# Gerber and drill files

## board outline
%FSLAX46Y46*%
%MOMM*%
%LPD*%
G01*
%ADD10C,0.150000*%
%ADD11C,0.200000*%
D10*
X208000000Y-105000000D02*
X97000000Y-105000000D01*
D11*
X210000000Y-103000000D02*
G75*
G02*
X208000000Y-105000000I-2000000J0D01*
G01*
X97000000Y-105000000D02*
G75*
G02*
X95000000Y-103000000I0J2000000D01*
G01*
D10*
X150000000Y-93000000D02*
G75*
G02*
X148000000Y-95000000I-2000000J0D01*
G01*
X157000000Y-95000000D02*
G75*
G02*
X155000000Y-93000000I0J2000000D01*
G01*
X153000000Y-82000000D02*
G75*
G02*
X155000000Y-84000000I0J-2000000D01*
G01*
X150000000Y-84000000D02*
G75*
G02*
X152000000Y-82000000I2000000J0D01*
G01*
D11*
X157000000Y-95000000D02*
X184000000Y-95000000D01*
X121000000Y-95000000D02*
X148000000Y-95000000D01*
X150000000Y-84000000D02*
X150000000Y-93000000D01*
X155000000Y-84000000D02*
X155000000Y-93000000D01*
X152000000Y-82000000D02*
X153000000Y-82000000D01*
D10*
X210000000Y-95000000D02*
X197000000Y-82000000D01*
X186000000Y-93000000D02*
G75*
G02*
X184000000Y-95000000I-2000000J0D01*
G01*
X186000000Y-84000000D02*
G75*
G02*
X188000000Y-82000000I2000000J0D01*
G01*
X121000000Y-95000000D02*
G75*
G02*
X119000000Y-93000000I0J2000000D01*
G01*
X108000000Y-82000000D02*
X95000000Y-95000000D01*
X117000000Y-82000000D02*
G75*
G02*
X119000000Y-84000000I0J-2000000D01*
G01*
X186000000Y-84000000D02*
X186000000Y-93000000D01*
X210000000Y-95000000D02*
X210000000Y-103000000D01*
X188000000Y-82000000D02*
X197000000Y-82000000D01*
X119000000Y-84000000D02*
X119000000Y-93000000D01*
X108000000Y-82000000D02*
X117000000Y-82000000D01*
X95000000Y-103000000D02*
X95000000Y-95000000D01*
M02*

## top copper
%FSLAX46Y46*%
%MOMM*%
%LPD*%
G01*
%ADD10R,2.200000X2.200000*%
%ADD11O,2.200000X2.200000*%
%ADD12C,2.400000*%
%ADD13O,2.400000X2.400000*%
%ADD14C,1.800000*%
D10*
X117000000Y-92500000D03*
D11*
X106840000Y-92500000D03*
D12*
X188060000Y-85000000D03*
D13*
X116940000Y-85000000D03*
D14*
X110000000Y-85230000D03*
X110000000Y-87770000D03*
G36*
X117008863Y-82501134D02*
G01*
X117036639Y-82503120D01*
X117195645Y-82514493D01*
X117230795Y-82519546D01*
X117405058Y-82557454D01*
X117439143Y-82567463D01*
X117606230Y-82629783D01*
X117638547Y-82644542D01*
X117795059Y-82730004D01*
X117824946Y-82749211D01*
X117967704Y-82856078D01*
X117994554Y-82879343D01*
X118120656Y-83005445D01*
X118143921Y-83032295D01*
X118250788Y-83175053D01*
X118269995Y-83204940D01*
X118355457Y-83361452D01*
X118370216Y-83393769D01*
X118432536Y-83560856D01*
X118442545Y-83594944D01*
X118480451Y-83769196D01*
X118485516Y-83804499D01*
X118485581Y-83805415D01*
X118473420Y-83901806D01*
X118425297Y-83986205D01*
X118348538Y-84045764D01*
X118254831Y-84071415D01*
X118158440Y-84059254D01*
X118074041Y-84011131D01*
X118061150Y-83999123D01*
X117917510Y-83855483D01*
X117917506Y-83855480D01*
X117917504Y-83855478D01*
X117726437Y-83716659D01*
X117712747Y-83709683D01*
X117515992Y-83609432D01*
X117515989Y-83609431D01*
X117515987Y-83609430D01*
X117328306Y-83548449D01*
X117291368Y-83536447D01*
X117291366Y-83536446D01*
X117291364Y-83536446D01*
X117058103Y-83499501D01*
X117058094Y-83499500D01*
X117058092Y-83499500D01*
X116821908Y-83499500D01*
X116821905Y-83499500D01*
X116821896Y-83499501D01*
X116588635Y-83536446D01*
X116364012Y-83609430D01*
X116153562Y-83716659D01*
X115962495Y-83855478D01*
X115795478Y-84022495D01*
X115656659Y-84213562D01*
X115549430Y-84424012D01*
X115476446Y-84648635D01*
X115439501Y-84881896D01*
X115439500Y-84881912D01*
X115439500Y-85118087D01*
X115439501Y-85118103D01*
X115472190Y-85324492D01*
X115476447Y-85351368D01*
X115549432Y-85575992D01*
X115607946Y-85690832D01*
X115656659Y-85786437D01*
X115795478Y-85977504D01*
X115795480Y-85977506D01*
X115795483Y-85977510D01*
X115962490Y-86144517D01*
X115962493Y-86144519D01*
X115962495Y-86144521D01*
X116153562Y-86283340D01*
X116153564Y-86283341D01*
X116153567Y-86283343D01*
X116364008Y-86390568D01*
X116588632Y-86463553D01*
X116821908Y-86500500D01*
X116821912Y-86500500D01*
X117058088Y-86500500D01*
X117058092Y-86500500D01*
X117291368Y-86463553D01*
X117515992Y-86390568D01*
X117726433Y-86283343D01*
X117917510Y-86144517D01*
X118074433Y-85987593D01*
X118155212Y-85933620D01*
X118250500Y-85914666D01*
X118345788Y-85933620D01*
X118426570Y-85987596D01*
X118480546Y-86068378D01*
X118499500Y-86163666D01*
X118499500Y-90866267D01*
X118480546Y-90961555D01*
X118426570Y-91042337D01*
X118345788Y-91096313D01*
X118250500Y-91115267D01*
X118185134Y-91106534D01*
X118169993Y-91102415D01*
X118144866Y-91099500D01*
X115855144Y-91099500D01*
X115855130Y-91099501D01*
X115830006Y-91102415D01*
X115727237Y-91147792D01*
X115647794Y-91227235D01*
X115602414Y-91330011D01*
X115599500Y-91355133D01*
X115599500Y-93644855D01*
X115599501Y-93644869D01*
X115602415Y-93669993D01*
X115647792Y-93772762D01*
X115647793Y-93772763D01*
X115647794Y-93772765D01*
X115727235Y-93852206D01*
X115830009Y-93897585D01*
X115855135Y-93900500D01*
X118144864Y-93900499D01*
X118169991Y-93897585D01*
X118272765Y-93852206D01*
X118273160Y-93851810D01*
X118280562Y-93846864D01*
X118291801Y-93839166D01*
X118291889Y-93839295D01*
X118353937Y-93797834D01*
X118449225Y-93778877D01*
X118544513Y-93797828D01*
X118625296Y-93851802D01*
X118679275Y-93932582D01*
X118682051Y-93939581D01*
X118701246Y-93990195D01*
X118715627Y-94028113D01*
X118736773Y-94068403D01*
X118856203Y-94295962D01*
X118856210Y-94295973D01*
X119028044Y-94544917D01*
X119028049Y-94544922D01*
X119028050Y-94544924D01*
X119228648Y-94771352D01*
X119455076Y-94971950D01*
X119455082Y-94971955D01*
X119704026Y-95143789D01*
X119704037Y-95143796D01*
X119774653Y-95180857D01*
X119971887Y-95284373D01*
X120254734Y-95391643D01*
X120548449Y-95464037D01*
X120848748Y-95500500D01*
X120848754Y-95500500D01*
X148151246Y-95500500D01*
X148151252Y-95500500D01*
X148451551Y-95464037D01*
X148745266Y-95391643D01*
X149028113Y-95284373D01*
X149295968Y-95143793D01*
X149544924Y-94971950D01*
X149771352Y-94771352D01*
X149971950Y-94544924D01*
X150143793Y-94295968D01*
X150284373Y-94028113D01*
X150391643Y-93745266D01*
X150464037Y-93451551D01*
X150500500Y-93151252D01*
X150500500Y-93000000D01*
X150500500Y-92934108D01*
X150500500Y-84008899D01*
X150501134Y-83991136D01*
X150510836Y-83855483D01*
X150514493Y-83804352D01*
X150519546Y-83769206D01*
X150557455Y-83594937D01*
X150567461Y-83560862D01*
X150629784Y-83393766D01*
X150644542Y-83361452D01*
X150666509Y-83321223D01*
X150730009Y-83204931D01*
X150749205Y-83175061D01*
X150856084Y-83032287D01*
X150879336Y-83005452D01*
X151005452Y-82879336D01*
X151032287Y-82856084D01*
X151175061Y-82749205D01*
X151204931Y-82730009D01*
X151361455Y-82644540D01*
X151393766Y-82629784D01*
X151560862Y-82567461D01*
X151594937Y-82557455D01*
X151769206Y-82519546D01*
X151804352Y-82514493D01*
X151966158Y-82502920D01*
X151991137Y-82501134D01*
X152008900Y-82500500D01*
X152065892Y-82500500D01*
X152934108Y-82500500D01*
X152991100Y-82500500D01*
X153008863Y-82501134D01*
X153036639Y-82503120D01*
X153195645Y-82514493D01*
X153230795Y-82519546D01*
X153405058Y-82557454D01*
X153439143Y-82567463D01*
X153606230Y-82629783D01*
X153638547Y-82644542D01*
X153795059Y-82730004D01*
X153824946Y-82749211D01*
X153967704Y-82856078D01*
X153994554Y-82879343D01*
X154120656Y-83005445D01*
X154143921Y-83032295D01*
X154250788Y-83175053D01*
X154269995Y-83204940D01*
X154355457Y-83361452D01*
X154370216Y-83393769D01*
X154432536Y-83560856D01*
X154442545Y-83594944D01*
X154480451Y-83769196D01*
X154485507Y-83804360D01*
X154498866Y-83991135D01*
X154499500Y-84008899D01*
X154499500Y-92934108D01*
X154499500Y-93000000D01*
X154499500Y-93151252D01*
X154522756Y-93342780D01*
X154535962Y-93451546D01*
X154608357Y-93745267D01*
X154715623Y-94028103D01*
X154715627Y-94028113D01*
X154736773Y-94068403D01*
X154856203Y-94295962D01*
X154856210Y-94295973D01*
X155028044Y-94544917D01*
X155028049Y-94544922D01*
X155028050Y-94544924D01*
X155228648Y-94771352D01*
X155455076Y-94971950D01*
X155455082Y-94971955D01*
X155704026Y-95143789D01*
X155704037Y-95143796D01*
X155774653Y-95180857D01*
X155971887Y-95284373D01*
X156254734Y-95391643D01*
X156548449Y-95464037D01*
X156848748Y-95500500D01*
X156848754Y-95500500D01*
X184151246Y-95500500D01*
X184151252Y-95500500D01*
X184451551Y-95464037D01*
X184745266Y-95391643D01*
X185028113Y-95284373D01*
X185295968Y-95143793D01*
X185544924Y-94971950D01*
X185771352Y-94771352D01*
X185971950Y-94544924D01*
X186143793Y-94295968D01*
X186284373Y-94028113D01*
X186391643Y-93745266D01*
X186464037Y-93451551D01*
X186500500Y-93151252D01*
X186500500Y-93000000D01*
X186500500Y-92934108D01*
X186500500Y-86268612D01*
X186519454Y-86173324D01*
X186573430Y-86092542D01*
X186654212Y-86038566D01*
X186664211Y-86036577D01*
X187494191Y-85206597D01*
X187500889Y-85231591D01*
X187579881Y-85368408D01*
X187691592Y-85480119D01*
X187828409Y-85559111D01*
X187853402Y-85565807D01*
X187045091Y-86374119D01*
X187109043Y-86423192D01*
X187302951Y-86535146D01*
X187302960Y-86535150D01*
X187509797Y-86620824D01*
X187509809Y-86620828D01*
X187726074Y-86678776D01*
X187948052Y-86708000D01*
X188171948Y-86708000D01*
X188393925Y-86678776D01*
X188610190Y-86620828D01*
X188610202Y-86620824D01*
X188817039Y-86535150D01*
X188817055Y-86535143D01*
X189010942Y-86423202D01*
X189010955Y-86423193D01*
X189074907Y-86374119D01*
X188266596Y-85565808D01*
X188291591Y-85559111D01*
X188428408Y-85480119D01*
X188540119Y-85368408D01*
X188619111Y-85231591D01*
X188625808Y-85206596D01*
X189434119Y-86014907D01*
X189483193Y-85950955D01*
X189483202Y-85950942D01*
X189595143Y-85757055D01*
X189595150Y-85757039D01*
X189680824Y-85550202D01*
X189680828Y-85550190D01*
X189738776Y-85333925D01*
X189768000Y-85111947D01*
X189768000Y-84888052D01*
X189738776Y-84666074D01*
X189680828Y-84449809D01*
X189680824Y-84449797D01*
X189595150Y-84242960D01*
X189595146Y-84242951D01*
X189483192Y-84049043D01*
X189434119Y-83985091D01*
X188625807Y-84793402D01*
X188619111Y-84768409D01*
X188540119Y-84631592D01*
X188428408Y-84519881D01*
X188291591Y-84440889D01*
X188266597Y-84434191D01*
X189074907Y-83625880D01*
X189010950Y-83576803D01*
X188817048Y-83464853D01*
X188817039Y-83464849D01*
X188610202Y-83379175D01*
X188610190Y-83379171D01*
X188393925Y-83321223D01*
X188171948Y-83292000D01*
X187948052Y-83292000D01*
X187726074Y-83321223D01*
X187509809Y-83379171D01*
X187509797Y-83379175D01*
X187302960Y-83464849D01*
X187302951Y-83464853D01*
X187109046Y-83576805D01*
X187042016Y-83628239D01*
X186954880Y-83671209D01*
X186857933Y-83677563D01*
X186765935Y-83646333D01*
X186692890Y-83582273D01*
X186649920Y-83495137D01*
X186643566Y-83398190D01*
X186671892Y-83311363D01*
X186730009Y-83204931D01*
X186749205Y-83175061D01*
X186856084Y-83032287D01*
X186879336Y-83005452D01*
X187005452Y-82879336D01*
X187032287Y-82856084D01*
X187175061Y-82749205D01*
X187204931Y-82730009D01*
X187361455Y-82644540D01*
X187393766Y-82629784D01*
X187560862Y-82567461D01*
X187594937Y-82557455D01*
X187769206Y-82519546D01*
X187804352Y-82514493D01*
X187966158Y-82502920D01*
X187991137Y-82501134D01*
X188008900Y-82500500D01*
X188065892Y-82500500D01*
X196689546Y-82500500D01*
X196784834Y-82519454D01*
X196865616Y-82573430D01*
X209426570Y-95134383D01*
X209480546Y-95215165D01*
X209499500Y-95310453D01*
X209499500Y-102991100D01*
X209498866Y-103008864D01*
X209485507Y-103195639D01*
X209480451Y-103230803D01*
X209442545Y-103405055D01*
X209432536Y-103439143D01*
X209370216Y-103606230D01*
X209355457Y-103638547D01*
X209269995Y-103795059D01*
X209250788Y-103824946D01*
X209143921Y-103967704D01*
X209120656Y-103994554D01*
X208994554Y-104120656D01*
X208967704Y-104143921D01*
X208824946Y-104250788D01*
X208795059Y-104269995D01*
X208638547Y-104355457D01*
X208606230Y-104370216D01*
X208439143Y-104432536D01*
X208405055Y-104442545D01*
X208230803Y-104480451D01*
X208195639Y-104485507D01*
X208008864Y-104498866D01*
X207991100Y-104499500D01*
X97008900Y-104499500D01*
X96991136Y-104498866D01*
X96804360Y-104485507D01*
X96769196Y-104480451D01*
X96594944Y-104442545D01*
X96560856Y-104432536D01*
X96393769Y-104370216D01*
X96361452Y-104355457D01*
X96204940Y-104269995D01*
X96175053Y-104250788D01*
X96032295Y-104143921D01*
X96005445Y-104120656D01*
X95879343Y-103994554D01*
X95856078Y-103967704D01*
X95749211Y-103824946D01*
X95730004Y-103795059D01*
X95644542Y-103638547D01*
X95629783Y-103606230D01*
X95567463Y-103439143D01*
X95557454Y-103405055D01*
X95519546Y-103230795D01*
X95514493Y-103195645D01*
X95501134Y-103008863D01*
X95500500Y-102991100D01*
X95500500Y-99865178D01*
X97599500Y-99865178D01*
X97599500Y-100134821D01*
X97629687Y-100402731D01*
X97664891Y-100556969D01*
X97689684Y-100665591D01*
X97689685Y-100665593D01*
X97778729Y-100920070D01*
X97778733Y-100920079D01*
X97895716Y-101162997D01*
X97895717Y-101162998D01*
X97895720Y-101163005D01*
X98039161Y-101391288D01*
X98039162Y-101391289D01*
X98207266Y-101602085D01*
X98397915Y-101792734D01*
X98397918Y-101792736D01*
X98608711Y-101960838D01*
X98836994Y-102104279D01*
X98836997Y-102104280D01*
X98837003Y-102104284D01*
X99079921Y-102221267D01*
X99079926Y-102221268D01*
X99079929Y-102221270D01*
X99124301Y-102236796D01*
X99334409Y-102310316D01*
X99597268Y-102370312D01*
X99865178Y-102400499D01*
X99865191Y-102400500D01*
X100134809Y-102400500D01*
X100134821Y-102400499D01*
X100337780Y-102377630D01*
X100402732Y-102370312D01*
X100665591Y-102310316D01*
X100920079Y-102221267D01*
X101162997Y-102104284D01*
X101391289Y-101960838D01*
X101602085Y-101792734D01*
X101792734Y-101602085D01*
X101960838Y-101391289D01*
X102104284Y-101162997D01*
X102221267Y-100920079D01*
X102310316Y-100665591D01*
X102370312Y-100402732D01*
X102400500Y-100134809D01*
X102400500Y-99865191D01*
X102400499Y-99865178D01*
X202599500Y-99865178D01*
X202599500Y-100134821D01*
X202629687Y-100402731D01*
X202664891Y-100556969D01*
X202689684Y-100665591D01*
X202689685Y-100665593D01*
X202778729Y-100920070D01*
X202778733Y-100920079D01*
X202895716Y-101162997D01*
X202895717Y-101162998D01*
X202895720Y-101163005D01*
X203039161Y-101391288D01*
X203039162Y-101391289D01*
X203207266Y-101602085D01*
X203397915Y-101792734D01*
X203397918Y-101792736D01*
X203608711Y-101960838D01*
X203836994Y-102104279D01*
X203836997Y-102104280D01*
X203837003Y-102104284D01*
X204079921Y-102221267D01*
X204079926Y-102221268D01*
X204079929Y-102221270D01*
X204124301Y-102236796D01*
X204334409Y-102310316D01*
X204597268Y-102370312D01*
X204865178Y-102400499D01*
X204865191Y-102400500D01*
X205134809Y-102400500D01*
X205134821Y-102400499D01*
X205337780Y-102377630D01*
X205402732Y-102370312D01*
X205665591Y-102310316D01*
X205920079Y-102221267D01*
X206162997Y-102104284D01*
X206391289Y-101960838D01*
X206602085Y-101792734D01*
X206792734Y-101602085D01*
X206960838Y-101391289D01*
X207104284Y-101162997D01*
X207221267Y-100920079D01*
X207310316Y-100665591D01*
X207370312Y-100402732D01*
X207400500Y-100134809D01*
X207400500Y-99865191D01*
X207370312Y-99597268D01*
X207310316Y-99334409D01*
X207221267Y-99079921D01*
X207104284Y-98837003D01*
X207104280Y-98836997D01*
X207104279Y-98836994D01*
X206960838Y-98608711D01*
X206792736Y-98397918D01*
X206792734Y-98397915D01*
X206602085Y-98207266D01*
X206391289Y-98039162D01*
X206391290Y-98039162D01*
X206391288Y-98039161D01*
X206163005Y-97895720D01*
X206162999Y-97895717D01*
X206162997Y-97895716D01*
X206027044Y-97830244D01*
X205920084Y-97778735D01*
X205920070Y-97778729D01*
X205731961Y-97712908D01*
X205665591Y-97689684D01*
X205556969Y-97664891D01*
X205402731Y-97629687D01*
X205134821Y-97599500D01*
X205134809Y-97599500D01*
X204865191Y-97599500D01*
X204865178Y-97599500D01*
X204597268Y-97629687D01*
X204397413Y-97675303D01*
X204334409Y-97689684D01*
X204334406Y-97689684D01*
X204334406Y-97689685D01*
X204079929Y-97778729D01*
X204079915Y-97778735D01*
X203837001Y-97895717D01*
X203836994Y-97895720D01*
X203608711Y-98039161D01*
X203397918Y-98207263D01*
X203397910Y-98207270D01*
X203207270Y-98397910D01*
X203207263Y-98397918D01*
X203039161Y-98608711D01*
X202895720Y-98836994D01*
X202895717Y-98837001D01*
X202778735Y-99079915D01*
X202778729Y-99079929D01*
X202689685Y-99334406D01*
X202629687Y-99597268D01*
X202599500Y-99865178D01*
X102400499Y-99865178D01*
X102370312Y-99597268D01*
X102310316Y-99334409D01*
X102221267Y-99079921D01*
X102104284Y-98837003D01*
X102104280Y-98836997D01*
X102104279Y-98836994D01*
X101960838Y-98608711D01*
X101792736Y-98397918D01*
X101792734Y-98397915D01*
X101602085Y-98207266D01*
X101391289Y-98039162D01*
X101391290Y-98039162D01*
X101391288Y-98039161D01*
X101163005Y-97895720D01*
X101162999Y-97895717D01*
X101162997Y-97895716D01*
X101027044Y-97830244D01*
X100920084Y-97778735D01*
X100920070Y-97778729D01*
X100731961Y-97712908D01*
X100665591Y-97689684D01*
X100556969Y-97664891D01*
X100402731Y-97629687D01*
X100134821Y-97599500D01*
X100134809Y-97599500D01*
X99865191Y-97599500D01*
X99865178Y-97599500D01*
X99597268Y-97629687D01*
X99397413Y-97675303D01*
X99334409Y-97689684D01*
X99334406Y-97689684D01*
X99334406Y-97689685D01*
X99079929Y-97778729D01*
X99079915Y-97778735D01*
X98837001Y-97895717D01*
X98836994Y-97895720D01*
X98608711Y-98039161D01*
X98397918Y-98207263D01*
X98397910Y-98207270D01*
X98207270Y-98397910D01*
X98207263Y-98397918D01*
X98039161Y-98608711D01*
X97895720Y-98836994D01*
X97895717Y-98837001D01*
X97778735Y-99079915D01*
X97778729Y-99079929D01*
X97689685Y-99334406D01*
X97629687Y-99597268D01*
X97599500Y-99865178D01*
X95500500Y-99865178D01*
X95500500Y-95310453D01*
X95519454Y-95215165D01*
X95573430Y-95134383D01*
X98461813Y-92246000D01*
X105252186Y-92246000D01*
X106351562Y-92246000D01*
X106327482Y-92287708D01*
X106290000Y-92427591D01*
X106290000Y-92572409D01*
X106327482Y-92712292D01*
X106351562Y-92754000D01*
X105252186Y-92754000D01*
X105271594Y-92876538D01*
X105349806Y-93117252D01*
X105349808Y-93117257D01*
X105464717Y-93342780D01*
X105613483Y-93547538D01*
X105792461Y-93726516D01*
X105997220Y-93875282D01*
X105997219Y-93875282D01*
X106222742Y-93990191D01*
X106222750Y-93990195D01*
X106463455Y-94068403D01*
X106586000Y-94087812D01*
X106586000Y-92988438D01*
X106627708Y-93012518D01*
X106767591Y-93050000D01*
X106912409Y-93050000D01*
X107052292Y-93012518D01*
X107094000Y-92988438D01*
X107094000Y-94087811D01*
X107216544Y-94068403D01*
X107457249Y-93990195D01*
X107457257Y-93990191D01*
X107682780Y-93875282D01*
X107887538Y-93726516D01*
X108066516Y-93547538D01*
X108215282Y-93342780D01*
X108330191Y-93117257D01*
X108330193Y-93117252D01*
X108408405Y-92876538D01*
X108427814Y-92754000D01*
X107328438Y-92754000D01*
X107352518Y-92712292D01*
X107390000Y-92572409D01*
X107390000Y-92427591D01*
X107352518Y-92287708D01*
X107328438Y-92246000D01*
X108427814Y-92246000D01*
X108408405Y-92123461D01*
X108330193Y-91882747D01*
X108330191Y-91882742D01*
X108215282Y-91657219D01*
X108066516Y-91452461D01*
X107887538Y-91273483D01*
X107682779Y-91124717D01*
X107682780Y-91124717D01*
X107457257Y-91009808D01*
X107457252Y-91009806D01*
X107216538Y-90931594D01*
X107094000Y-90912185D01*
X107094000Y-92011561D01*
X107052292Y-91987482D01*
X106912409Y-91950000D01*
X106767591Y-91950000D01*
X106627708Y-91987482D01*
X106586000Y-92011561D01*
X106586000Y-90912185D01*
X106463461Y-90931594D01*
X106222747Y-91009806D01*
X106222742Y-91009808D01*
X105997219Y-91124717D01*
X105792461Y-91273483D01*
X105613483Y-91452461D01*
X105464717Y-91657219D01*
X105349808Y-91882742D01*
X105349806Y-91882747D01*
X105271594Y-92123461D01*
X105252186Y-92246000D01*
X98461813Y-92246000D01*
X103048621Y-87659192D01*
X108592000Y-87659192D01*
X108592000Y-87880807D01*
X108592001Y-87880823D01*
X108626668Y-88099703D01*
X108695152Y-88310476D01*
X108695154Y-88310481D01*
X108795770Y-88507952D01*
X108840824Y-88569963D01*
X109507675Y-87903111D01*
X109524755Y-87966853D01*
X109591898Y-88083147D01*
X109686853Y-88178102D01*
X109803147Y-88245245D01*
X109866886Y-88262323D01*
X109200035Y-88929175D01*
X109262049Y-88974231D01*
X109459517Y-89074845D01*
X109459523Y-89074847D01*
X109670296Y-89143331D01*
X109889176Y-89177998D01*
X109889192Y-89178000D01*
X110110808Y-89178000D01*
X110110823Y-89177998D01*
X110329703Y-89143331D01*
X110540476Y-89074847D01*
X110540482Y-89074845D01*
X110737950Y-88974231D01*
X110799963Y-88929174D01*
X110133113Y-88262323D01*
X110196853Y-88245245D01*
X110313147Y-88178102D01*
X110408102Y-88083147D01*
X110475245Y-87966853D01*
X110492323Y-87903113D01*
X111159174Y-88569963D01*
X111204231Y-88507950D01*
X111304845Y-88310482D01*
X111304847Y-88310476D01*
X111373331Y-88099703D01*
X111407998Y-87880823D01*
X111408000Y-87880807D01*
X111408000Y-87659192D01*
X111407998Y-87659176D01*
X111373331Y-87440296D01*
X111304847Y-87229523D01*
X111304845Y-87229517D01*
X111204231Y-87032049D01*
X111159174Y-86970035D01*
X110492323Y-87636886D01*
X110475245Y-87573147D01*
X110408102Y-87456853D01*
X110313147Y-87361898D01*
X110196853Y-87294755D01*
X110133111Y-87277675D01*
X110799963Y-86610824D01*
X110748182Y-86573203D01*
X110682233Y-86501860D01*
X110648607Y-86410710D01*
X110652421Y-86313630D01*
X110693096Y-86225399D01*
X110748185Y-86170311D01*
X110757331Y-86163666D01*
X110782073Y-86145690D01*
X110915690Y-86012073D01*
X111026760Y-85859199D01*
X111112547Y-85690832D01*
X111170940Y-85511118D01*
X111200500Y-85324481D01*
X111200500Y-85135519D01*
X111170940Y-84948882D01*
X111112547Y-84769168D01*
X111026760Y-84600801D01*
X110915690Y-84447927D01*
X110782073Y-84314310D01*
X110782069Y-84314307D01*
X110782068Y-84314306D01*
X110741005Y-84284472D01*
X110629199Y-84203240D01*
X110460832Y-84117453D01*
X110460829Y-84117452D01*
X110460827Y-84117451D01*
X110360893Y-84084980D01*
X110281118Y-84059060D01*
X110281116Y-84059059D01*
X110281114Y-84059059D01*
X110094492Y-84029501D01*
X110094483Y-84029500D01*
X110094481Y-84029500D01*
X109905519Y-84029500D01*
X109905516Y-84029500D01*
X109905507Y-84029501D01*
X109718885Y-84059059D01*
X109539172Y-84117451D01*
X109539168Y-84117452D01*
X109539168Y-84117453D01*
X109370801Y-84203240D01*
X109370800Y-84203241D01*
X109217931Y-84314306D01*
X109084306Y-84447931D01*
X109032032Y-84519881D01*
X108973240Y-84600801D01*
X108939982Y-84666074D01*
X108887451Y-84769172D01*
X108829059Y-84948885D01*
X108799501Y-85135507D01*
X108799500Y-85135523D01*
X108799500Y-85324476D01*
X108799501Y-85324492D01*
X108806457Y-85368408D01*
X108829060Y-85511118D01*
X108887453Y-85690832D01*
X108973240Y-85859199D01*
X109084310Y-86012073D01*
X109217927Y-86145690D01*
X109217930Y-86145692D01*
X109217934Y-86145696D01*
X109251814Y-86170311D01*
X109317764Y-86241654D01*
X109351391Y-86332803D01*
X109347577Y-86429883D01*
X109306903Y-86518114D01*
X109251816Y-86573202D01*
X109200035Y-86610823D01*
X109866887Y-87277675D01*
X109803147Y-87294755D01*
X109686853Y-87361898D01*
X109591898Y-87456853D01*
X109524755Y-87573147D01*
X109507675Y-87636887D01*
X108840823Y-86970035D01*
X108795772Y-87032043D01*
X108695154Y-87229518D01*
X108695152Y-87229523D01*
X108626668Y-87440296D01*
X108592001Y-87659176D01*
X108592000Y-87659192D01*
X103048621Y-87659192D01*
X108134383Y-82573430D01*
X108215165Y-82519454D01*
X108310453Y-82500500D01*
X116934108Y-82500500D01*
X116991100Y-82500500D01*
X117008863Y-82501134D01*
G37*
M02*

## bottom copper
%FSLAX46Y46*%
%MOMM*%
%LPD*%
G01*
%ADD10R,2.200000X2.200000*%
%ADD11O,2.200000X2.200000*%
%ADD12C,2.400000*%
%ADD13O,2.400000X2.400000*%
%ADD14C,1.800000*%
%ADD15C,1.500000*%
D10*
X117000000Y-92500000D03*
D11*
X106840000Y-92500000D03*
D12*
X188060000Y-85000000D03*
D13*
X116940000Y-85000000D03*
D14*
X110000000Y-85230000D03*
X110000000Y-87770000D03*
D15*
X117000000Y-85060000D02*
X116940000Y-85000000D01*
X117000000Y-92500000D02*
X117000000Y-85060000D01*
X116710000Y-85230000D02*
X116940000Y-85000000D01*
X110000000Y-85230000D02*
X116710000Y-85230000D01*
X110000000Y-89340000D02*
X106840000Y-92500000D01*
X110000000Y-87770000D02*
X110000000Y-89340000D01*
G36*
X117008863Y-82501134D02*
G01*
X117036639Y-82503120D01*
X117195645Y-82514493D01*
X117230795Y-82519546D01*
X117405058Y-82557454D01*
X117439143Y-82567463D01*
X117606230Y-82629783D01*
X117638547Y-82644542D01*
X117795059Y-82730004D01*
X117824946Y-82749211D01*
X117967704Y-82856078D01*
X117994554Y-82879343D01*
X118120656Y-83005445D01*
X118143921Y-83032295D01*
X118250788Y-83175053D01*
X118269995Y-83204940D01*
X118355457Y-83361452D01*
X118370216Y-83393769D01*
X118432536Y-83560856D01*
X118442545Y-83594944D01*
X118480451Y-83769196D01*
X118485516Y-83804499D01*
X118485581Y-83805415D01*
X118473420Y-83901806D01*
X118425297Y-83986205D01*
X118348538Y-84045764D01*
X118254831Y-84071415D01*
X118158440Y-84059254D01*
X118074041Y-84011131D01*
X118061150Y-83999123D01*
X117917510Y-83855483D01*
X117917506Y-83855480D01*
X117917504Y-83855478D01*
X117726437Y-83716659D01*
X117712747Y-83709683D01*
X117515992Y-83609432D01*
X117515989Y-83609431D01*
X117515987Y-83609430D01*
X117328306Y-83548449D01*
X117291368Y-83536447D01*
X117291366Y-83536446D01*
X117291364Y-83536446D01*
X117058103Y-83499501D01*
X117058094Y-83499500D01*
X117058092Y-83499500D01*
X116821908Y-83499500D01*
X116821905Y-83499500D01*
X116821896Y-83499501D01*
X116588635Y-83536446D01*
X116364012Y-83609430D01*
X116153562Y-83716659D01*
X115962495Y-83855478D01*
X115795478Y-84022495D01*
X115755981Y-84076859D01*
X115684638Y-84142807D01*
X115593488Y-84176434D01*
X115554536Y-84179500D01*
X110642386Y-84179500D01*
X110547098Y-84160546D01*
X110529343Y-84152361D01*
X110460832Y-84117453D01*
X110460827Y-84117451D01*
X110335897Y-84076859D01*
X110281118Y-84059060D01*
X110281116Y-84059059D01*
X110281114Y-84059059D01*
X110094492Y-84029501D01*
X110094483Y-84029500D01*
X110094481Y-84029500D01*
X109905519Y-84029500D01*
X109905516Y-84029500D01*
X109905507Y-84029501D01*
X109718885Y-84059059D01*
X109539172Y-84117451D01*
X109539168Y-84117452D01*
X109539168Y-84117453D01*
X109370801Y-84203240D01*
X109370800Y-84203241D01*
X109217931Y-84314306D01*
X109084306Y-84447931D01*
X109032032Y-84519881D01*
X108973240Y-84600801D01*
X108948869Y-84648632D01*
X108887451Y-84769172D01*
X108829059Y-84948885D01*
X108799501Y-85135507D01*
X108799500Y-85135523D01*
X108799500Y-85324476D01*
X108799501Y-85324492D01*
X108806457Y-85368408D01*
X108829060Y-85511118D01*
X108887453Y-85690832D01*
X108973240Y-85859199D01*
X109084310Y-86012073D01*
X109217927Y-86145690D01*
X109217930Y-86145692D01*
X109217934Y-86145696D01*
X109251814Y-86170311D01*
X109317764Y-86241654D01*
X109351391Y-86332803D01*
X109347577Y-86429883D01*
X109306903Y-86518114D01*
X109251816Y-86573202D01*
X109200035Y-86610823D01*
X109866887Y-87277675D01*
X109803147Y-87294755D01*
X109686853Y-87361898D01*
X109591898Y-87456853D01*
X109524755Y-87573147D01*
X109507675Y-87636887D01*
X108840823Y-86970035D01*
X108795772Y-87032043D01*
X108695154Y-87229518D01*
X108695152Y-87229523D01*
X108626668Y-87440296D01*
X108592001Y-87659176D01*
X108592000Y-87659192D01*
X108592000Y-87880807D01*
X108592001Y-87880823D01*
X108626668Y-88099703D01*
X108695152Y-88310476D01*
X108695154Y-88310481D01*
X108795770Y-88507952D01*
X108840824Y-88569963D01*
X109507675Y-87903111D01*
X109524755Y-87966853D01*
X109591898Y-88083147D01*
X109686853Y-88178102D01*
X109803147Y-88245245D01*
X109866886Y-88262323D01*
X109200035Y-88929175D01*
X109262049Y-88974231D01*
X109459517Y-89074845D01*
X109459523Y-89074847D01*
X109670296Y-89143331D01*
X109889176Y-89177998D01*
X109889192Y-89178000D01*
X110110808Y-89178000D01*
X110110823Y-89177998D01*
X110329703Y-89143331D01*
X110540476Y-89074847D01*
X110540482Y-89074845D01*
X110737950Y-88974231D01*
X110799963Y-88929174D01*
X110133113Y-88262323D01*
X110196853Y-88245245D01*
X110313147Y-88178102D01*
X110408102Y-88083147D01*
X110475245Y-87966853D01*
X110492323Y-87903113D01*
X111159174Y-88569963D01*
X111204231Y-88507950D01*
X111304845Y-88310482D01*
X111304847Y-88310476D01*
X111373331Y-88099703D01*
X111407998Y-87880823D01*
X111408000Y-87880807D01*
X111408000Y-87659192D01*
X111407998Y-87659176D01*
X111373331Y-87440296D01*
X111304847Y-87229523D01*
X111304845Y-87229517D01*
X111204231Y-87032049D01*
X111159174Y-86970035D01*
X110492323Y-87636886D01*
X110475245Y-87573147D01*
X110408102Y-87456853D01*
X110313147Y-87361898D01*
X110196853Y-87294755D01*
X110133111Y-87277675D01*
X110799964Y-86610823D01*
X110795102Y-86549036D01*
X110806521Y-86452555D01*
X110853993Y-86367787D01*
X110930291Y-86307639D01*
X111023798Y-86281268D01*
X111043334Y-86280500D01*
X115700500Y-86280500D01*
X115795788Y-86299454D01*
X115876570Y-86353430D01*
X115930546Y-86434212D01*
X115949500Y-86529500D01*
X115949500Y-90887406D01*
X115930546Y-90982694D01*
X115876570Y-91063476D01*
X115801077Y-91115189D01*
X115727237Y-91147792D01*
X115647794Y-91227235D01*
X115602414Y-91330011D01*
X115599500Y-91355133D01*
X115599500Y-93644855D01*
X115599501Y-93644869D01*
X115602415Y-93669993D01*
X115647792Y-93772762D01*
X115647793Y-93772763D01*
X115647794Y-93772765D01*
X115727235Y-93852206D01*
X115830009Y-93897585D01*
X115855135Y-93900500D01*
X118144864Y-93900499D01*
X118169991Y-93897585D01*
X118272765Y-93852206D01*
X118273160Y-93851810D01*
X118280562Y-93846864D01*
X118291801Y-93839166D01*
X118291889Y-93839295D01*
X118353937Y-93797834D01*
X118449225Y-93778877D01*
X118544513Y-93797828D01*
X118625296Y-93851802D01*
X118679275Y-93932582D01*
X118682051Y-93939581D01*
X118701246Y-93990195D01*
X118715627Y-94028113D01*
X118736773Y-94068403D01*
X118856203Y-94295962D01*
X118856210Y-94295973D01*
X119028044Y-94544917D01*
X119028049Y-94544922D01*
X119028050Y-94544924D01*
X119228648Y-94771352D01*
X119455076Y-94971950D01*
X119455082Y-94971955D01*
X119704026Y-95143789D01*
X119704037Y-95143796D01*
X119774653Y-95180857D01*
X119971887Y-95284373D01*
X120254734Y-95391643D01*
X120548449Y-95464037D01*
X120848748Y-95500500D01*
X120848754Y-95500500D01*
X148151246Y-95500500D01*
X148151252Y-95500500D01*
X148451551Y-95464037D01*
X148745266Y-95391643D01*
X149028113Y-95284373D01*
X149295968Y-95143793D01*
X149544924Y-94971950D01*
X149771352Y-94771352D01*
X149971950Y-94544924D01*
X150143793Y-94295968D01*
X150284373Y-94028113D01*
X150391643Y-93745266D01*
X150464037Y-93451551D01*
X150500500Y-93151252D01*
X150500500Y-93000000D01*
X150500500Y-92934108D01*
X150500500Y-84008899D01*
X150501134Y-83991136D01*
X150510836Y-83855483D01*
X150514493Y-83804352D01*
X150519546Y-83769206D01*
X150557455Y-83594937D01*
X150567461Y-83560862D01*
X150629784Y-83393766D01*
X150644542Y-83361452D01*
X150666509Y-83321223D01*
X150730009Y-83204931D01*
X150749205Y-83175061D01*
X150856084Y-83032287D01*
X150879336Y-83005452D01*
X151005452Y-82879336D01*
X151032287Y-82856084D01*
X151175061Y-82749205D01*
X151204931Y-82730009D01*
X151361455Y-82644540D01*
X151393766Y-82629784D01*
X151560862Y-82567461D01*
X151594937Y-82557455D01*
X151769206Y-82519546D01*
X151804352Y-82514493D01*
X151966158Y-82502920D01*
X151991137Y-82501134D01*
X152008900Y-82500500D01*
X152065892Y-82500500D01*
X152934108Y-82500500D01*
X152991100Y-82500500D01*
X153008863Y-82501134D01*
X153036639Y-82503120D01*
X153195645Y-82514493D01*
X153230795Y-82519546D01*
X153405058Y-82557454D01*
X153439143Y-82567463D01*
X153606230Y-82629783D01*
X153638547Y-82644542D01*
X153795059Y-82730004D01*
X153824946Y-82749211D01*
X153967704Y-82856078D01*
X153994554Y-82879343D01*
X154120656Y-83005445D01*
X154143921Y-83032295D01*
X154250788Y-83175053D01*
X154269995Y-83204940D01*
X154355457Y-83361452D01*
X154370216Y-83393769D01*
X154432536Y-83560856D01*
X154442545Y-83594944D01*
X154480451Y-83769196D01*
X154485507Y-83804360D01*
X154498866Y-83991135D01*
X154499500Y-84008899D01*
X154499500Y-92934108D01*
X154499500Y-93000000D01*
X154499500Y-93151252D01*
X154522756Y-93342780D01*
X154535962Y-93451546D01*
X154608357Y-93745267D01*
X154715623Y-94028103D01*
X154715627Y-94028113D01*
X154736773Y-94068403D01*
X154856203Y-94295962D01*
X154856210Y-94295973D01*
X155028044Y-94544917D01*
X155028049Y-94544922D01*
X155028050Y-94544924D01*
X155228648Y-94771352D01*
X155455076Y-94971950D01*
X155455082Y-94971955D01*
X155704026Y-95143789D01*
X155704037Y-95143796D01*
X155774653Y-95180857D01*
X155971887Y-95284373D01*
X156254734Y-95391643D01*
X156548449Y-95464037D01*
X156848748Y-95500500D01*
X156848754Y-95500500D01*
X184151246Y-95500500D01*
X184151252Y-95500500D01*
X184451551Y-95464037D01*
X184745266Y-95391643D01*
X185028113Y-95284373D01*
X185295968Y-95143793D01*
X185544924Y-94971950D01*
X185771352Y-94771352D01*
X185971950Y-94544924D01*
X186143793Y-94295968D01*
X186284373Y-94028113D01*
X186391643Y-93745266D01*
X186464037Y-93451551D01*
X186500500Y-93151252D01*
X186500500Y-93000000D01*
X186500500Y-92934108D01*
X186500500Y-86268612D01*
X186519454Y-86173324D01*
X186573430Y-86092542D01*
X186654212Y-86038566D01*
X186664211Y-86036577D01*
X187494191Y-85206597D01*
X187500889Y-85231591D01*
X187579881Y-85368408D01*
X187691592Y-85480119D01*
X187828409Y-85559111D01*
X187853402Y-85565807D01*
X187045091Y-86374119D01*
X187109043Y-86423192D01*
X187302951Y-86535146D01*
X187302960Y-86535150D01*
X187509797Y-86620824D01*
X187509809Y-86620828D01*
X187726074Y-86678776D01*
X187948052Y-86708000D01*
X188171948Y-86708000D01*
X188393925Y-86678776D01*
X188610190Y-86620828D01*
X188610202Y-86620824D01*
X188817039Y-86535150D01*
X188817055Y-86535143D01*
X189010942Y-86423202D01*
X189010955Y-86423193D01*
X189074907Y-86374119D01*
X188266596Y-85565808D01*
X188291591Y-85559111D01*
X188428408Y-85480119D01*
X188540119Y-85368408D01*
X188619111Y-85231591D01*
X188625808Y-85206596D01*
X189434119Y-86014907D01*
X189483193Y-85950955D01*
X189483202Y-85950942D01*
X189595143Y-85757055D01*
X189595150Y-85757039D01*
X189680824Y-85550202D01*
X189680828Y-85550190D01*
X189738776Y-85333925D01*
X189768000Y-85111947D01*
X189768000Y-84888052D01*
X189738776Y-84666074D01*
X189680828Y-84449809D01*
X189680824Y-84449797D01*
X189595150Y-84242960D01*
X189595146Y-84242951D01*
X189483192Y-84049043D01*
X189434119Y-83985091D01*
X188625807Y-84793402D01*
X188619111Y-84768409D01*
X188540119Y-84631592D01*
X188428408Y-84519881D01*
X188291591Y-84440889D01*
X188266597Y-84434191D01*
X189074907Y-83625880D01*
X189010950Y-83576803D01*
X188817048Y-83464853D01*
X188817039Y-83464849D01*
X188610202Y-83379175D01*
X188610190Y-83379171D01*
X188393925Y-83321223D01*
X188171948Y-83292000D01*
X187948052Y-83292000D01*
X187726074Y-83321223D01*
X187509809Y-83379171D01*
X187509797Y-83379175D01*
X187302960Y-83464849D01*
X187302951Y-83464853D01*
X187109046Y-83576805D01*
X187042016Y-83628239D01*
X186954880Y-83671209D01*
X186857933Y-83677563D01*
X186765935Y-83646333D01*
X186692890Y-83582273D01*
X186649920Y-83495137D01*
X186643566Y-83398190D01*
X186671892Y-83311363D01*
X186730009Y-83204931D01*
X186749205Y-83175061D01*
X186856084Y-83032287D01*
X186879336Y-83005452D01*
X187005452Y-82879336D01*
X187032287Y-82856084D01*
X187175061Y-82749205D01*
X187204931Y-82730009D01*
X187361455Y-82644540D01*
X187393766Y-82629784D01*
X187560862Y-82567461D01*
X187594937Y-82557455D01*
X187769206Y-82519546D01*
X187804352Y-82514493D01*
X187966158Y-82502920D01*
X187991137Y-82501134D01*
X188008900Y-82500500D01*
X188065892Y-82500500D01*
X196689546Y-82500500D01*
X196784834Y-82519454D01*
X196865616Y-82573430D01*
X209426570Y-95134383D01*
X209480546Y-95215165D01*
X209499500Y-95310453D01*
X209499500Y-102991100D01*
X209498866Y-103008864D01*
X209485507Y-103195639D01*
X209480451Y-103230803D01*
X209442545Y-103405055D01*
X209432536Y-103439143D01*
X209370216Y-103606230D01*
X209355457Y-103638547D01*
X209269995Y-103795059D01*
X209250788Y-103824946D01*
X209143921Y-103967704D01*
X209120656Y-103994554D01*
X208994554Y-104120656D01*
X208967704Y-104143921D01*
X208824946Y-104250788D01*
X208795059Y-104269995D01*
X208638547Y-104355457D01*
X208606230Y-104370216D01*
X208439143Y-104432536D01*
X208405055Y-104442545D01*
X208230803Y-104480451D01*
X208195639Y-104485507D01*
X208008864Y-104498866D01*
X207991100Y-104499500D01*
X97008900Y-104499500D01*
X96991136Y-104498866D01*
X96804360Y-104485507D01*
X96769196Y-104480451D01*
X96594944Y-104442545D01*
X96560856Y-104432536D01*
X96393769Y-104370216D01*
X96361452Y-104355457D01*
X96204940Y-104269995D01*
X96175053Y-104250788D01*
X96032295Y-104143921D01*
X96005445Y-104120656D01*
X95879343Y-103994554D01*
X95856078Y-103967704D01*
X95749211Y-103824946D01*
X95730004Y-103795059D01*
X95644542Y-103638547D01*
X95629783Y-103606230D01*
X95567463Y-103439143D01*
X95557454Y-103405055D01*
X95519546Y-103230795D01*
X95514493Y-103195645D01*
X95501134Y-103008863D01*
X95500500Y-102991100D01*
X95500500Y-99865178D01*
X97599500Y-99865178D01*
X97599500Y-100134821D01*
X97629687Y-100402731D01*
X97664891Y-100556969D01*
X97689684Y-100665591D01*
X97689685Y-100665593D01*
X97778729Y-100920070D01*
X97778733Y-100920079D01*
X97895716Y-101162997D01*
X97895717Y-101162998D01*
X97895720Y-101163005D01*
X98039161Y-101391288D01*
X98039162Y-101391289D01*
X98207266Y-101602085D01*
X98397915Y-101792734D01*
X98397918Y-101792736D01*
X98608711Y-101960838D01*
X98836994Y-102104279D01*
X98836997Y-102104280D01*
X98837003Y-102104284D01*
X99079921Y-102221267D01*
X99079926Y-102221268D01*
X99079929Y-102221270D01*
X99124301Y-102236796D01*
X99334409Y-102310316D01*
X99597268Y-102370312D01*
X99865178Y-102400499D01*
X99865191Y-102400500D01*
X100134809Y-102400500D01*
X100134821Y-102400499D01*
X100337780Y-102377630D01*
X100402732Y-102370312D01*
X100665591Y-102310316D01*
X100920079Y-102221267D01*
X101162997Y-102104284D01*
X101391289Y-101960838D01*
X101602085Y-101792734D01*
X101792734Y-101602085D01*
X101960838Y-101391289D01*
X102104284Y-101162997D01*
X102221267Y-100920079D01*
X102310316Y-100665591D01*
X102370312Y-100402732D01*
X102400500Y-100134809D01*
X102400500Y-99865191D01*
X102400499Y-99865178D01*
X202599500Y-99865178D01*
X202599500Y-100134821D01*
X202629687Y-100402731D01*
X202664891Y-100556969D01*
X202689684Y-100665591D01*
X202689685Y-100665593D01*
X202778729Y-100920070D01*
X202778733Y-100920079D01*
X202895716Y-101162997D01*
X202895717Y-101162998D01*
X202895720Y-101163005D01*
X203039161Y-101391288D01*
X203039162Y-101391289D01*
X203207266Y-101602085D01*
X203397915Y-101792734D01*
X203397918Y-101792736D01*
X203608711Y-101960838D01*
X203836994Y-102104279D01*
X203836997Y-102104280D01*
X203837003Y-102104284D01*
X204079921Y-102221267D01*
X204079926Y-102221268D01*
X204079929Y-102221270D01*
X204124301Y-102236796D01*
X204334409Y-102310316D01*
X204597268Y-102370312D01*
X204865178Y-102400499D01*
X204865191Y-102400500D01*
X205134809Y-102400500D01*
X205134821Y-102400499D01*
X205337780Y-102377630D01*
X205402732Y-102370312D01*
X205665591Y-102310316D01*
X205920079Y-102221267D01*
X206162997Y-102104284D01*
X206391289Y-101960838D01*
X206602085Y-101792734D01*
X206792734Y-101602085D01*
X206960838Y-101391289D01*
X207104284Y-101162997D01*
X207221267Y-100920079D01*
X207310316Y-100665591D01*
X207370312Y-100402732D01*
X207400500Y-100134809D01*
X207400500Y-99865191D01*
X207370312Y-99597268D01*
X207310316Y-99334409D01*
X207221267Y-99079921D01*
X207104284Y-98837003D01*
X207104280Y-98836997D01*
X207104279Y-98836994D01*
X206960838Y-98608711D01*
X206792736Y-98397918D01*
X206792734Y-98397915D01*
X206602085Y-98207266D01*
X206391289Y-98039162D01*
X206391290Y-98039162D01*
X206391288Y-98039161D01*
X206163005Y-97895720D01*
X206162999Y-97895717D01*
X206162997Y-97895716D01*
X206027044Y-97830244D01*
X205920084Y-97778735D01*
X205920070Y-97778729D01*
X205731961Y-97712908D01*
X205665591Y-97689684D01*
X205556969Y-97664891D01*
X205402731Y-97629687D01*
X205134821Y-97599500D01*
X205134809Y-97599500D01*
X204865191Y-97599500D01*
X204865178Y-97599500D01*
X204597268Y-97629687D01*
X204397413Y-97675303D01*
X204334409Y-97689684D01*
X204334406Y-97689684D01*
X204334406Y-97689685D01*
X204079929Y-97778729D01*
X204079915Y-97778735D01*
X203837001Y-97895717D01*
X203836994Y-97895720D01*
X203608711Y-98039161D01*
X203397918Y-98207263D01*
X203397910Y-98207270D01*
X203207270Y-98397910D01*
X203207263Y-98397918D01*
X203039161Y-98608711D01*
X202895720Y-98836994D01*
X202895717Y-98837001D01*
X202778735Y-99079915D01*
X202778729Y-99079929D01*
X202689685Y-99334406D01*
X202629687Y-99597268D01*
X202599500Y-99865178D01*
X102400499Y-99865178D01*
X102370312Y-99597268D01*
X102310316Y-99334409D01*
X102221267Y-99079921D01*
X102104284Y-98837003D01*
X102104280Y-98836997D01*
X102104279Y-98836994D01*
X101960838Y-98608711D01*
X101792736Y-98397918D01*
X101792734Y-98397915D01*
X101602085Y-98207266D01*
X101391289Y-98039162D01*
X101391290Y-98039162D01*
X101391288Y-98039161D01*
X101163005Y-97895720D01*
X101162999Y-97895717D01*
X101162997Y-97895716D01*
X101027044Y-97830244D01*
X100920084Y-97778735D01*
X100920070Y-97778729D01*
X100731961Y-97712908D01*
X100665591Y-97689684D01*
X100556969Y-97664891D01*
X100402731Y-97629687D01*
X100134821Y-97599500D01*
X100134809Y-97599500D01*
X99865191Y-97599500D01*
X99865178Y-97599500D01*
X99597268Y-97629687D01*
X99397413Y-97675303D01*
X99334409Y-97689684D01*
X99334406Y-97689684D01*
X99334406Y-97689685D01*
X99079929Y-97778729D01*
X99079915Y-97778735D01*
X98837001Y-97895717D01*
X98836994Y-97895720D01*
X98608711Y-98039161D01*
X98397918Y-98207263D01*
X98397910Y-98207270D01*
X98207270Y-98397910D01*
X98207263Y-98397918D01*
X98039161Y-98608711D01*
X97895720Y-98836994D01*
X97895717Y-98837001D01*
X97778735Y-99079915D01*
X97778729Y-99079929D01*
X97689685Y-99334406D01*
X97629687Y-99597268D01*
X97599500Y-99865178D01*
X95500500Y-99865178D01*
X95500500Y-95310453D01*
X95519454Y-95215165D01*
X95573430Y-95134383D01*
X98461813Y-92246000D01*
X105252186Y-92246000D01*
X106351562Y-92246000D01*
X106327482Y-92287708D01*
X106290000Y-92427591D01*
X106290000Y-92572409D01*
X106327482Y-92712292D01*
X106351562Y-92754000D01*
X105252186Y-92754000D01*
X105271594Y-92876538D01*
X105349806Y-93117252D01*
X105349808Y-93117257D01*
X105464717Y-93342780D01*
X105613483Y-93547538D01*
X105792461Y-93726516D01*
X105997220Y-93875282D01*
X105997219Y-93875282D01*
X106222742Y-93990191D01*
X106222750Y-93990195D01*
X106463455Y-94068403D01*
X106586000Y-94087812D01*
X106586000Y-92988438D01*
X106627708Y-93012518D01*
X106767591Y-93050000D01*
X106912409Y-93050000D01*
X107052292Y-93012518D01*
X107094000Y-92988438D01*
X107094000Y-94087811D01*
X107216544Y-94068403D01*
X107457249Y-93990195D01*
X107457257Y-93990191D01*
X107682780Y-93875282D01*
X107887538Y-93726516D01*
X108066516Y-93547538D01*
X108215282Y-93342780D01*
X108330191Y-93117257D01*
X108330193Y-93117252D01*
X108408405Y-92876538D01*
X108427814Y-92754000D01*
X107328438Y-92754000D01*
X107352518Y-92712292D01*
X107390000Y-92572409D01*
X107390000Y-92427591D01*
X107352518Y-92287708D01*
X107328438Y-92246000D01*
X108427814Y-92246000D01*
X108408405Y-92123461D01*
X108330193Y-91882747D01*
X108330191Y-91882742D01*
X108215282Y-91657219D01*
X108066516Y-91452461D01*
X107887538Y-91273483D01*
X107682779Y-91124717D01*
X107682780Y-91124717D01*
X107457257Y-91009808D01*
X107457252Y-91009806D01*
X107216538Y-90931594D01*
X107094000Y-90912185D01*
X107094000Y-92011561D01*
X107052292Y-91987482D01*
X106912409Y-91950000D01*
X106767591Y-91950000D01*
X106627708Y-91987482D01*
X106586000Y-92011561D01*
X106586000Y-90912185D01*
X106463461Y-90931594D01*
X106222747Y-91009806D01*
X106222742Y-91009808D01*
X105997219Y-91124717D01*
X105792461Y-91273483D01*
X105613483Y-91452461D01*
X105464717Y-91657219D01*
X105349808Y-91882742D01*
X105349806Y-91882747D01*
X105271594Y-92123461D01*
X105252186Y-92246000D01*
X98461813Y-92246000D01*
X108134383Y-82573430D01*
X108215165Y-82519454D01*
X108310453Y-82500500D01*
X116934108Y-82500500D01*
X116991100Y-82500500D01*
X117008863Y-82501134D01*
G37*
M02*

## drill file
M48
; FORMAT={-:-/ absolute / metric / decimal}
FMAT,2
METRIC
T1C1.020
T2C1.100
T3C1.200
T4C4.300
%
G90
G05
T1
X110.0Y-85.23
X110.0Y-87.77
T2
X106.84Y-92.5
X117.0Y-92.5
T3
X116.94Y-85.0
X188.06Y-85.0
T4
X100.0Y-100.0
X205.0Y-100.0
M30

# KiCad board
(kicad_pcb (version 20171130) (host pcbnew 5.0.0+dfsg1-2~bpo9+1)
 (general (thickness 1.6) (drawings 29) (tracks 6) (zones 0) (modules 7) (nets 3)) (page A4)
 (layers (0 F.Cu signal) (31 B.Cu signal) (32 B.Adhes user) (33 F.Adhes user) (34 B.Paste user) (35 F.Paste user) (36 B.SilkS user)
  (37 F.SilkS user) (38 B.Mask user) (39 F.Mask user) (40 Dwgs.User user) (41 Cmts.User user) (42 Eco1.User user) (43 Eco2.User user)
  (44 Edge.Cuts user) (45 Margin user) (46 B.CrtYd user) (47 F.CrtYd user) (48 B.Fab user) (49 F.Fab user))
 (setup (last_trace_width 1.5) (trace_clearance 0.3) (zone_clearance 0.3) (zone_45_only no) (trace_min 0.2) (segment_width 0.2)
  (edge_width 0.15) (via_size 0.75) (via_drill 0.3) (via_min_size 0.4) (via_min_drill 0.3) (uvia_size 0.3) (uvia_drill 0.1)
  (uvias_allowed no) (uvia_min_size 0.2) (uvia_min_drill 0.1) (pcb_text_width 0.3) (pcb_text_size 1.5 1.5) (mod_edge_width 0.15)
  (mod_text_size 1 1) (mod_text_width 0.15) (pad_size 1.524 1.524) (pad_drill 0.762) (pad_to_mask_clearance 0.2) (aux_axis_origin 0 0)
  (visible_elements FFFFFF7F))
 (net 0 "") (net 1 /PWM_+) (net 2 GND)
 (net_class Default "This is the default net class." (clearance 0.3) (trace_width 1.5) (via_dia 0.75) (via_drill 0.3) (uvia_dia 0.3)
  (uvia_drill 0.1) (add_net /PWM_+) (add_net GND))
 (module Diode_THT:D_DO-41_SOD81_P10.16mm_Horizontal (layer F.Cu) (at 117 92.5 180)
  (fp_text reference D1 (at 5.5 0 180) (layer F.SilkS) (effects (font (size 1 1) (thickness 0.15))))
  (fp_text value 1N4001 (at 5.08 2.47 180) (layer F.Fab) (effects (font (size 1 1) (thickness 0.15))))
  (pad 1 thru_hole rect (at 0 0 180) (size 2.2 2.2) (drill 1.1) (layers *.Cu *.Mask) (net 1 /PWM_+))
  (pad 2 thru_hole oval (at 10.16 0 180) (size 2.2 2.2) (drill 1.1) (layers *.Cu *.Mask) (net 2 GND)))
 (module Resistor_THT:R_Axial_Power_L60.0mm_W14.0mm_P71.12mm (layer F.Cu) (at 152.5 85 180)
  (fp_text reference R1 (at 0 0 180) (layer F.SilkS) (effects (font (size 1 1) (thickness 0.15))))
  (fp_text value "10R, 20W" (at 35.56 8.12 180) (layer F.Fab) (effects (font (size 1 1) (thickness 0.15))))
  (pad 1 thru_hole circle (at -35.56 0 180) (size 2.4 2.4) (drill 1.2) (layers *.Cu *.Mask) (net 2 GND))
  (pad 2 thru_hole oval (at 35.56 0 180) (size 2.4 2.4) (drill 1.2) (layers *.Cu *.Mask) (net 1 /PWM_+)))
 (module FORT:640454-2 (layer F.Cu) (at 110 86.5 270)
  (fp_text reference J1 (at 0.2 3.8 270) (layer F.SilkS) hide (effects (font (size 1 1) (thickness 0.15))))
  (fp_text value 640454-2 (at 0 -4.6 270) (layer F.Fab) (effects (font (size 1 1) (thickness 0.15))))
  (pad 1 thru_hole circle (at -1.27 0 270) (size 1.8 1.8) (drill 1.02) (layers *.Cu *.Mask) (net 1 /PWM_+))
  (pad 2 thru_hole circle (at 1.27 0 270) (size 1.8 1.8) (drill 1.02) (layers *.Cu *.Mask) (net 2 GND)))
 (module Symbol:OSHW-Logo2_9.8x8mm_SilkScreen (layer F.Cu) (at 195 92.5)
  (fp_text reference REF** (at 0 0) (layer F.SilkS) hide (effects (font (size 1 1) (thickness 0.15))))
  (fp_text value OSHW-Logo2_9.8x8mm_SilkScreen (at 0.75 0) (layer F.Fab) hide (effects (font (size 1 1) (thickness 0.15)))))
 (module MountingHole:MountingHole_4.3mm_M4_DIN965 (layer F.Cu) (at 100 100)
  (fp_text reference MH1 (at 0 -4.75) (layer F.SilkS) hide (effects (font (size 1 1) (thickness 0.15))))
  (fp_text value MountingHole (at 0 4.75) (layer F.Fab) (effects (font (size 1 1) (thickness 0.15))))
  (pad 1 np_thru_hole circle (at 0 0) (size 4.3 4.3) (drill 4.3) (layers *.Cu *.Mask)))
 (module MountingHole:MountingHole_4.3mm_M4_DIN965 (layer F.Cu) (at 205 100)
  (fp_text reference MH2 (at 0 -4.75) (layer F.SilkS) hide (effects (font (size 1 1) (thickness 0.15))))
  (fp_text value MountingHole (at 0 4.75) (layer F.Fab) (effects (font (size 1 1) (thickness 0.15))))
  (pad 1 np_thru_hole circle (at 0 0) (size 4.3 4.3) (drill 4.3) (layers *.Cu *.Mask)))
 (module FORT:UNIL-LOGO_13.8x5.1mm (layer F.Cu) (at 195 100)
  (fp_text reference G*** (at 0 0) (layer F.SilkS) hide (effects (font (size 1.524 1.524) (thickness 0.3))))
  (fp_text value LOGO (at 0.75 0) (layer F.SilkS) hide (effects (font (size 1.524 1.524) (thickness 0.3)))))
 (gr_line (start 208 105) (end 97 105) (layer Edge.Cuts) (width 0.15))
 (gr_arc (start 208 103) (end 208 105) (angle -90) (layer Edge.Cuts) (width 0.2))
 (gr_arc (start 97 103) (end 95 103) (angle -90) (layer Edge.Cuts) (width 0.2))
 (gr_arc (start 148 93) (end 148 95) (angle -90) (layer Edge.Cuts) (width 0.15))
 (gr_arc (start 157 93) (end 155 93) (angle -90) (layer Edge.Cuts) (width 0.15))
 (gr_arc (start 153 84) (end 155 84) (angle -90) (layer Edge.Cuts) (width 0.15))
 (gr_arc (start 152 84) (end 152 82) (angle -90) (layer Edge.Cuts) (width 0.15))
 (gr_line (start 157 95) (end 184 95) (layer Edge.Cuts) (width 0.2))
 (gr_line (start 121 95) (end 148 95) (layer Edge.Cuts) (width 0.2))
 (gr_line (start 150 84) (end 150 93) (layer Edge.Cuts) (width 0.2))
 (gr_line (start 155 84) (end 155 93) (layer Edge.Cuts) (width 0.2))
 (gr_line (start 152 82) (end 153 82) (layer Edge.Cuts) (width 0.2))
 (gr_line (start 210 95) (end 197 82) (layer Edge.Cuts) (width 0.15))
 (gr_arc (start 184 93) (end 184 95) (angle -90) (layer Edge.Cuts) (width 0.15))
 (gr_arc (start 188 84) (end 188 82) (angle -90) (layer Edge.Cuts) (width 0.15))
 (gr_arc (start 121 93) (end 119 93) (angle -90) (layer Edge.Cuts) (width 0.15))
 (gr_line (start 108 82) (end 95 95) (layer Edge.Cuts) (width 0.15))
 (gr_arc (start 117 84) (end 119 84) (angle -90) (layer Edge.Cuts) (width 0.15))
 (gr_line (start 186 84) (end 186 93) (layer Edge.Cuts) (width 0.15))
 (gr_line (start 210 95) (end 210 103) (layer Edge.Cuts) (width 0.15))
 (gr_line (start 188 82) (end 197 82) (layer Edge.Cuts) (width 0.15))
 (gr_line (start 119 84) (end 119 93) (layer Edge.Cuts) (width 0.15))
 (gr_line (start 108 82) (end 117 82) (layer Edge.Cuts) (width 0.15))
 (gr_line (start 95 103) (end 95 95) (layer Edge.Cuts) (width 0.15))
 (segment (start 117 85.06) (end 116.94 85) (width 1.5) (layer B.Cu) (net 1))
 (segment (start 117 92.5) (end 117 85.06) (width 1.5) (layer B.Cu) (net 1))
 (segment (start 116.71 85.23) (end 116.94 85) (width 1.5) (layer B.Cu) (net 1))
 (segment (start 110 85.23) (end 116.71 85.23) (width 1.5) (layer B.Cu) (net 1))
 (segment (start 110 89.34) (end 106.84 92.5) (width 1.5) (layer B.Cu) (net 2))
 (segment (start 110 87.77) (end 110 89.34) (width 1.5) (layer B.Cu) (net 2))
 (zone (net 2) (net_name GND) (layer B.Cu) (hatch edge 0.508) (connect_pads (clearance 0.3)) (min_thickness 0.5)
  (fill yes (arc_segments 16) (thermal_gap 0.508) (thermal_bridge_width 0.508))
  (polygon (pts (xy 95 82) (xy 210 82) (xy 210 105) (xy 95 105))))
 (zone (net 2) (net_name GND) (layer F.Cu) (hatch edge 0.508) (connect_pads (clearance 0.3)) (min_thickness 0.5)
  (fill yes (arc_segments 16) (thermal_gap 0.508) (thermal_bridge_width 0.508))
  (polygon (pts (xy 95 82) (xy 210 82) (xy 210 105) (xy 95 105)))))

